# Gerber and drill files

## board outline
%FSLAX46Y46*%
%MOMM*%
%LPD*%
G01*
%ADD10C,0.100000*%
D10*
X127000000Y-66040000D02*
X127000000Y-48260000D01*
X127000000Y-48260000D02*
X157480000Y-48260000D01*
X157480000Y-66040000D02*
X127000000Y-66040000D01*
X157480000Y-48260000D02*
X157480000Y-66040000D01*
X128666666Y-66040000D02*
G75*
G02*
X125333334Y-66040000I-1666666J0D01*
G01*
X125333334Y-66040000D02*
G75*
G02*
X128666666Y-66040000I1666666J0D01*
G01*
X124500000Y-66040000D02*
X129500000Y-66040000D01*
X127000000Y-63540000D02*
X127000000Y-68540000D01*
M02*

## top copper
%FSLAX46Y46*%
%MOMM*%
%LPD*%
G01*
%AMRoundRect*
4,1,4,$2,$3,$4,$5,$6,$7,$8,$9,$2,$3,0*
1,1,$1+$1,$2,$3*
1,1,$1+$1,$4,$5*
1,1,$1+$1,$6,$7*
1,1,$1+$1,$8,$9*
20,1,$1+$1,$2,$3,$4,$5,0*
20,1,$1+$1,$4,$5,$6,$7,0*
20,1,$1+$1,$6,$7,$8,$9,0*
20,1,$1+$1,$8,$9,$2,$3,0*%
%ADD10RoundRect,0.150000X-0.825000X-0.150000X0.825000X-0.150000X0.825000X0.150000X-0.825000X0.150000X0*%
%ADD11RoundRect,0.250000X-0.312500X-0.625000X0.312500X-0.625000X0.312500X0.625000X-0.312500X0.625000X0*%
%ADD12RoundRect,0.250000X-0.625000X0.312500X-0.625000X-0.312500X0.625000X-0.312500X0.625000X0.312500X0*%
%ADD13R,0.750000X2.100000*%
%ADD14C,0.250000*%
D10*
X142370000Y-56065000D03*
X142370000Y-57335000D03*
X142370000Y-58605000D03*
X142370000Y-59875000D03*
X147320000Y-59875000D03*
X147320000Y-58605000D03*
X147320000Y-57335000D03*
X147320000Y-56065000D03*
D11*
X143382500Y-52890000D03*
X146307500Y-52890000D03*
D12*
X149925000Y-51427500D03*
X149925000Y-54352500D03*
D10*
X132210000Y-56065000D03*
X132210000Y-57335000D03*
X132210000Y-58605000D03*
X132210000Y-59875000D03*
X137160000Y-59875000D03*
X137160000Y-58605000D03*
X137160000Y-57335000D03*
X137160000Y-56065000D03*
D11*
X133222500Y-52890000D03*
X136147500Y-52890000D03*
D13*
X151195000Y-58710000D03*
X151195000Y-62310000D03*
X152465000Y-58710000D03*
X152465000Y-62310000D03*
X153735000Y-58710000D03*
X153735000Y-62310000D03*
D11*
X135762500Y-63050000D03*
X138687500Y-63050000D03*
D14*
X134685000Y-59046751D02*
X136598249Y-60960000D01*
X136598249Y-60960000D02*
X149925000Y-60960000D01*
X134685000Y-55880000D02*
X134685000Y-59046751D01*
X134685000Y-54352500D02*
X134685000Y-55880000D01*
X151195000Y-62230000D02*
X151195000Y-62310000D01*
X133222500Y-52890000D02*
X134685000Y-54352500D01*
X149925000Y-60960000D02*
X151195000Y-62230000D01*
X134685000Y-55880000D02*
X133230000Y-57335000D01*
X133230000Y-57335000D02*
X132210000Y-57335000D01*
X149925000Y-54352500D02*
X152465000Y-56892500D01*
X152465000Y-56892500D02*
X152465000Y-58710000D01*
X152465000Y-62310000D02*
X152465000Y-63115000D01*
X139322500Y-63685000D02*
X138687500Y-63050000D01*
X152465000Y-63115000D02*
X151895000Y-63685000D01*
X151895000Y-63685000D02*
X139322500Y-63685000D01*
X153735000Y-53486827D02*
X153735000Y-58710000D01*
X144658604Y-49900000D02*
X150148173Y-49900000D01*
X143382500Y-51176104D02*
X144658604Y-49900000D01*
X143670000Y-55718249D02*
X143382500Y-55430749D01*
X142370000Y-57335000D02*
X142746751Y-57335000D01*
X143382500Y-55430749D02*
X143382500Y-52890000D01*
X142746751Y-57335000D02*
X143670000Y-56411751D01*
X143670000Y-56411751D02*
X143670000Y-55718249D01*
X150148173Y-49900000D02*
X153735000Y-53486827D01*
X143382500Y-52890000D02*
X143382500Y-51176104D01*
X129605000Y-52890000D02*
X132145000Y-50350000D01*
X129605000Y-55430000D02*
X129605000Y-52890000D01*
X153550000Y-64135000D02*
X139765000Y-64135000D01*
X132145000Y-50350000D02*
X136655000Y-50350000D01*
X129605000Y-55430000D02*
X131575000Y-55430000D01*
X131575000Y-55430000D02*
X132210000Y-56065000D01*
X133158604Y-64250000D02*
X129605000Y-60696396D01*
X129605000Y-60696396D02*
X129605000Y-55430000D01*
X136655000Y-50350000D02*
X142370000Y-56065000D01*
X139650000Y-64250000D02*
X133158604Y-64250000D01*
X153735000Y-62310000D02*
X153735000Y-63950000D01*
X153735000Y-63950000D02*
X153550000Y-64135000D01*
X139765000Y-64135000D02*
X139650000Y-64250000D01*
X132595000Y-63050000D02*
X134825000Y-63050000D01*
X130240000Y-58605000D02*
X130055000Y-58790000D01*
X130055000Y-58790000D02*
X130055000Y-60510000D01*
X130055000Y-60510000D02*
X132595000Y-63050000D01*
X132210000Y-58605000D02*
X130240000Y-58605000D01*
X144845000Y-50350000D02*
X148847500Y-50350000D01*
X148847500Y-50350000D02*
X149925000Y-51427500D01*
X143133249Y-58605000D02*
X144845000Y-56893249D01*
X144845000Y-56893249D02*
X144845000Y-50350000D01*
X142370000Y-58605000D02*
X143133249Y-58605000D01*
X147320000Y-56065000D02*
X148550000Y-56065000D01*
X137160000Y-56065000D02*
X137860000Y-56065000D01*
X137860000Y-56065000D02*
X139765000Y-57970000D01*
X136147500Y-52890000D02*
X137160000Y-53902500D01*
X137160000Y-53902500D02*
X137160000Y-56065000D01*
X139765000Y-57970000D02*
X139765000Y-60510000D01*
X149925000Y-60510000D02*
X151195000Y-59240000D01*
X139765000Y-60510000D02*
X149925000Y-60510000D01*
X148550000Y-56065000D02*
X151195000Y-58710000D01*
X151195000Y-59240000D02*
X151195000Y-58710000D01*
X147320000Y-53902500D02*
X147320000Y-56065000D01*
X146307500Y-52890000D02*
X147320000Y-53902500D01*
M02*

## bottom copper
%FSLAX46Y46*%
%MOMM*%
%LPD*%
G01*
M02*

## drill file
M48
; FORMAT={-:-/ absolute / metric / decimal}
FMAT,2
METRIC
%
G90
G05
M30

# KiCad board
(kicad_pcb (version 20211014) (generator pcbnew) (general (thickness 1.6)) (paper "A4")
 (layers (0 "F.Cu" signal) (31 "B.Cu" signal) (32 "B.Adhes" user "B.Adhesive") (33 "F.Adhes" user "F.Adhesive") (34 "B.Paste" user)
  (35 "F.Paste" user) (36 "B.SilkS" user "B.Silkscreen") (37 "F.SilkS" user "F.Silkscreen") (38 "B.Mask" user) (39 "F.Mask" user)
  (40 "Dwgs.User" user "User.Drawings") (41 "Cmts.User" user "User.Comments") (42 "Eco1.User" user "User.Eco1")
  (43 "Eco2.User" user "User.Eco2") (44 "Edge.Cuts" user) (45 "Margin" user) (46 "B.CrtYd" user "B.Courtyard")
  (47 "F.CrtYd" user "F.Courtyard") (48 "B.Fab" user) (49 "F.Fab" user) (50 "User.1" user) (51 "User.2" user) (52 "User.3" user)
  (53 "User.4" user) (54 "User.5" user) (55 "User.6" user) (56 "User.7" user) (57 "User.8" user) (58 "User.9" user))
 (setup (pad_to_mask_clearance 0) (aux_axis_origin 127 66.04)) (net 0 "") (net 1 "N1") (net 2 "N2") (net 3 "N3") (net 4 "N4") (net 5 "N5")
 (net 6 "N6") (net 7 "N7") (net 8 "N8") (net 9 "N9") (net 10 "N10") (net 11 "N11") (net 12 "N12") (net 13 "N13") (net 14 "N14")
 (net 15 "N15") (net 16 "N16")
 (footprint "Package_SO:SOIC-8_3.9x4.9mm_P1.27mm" (layer "F.Cu") (at 144.845 57.97)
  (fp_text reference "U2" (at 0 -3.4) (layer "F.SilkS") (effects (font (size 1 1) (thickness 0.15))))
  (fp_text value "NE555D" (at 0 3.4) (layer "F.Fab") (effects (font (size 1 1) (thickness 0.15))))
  (pad "1" smd roundrect (at -2.475 -1.905) (size 1.95 0.6) (layers "F.Cu" "F.Paste" "F.Mask") (roundrect_rratio 0.25) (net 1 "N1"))
  (pad "2" smd roundrect (at -2.475 -0.635) (size 1.95 0.6) (layers "F.Cu" "F.Paste" "F.Mask") (roundrect_rratio 0.25) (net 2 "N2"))
  (pad "3" smd roundrect (at -2.475 0.635) (size 1.95 0.6) (layers "F.Cu" "F.Paste" "F.Mask") (roundrect_rratio 0.25) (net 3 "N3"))
  (pad "4" smd roundrect (at -2.475 1.905) (size 1.95 0.6) (layers "F.Cu" "F.Paste" "F.Mask") (roundrect_rratio 0.25) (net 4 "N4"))
  (pad "5" smd roundrect (at 2.475 1.905) (size 1.95 0.6) (layers "F.Cu" "F.Paste" "F.Mask") (roundrect_rratio 0.25) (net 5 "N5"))
  (pad "6" smd roundrect (at 2.475 0.635) (size 1.95 0.6) (layers "F.Cu" "F.Paste" "F.Mask") (roundrect_rratio 0.25) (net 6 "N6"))
  (pad "7" smd roundrect (at 2.475 -0.635) (size 1.95 0.6) (layers "F.Cu" "F.Paste" "F.Mask") (roundrect_rratio 0.25) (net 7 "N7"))
  (pad "8" smd roundrect (at 2.475 -1.905) (size 1.95 0.6) (layers "F.Cu" "F.Paste" "F.Mask") (roundrect_rratio 0.25) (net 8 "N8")))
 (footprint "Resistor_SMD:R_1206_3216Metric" (layer "F.Cu") (at 144.845 52.89)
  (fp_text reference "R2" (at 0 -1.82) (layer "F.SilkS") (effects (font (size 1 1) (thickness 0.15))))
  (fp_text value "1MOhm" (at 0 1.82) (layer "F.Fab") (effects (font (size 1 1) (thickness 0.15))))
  (pad "1" smd roundrect (at -1.4625 0) (size 1.125 1.75) (layers "F.Cu" "F.Paste" "F.Mask") (roundrect_rratio 0.222222) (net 2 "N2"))
  (pad "2" smd roundrect (at 1.4625 0) (size 1.125 1.75) (layers "F.Cu" "F.Paste" "F.Mask") (roundrect_rratio 0.222222) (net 8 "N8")))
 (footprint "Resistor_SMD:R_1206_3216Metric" (layer "F.Cu") (at 149.925 52.89 -90)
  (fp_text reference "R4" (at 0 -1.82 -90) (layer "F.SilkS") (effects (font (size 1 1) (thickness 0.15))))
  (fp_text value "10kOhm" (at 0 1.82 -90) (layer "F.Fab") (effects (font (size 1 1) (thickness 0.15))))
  (pad "1" smd roundrect (at -1.4625 0 270) (size 1.125 1.75) (layers "F.Cu" "F.Paste" "F.Mask") (roundrect_rratio 0.222222) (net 3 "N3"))
  (pad "2" smd roundrect (at 1.4625 0 270) (size 1.125 1.75) (layers "F.Cu" "F.Paste" "F.Mask") (roundrect_rratio 0.222222) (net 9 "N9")))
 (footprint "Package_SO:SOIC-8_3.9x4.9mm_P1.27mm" (layer "F.Cu") (at 134.685 57.97)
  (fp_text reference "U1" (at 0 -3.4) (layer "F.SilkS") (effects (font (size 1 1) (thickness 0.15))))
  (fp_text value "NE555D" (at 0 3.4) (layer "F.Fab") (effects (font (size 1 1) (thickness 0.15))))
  (pad "1" smd roundrect (at -2.475 -1.905) (size 1.95 0.6) (layers "F.Cu" "F.Paste" "F.Mask") (roundrect_rratio 0.25) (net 1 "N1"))
  (pad "2" smd roundrect (at -2.475 -0.635) (size 1.95 0.6) (layers "F.Cu" "F.Paste" "F.Mask") (roundrect_rratio 0.25) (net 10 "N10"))
  (pad "3" smd roundrect (at -2.475 0.635) (size 1.95 0.6) (layers "F.Cu" "F.Paste" "F.Mask") (roundrect_rratio 0.25) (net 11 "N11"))
  (pad "4" smd roundrect (at -2.475 1.905) (size 1.95 0.6) (layers "F.Cu" "F.Paste" "F.Mask") (roundrect_rratio 0.25) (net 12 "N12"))
  (pad "5" smd roundrect (at 2.475 1.905) (size 1.95 0.6) (layers "F.Cu" "F.Paste" "F.Mask") (roundrect_rratio 0.25) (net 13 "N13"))
  (pad "6" smd roundrect (at 2.475 0.635) (size 1.95 0.6) (layers "F.Cu" "F.Paste" "F.Mask") (roundrect_rratio 0.25) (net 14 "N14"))
  (pad "7" smd roundrect (at 2.475 -0.635) (size 1.95 0.6) (layers "F.Cu" "F.Paste" "F.Mask") (roundrect_rratio 0.25) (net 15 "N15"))
  (pad "8" smd roundrect (at 2.475 -1.905) (size 1.95 0.6) (layers "F.Cu" "F.Paste" "F.Mask") (roundrect_rratio 0.25) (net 8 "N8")))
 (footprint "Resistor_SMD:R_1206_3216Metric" (layer "F.Cu") (at 134.685 52.89)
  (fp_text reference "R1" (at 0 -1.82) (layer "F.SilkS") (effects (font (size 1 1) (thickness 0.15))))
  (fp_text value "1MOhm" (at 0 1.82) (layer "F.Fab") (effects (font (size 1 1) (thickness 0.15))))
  (pad "1" smd roundrect (at -1.4625 0) (size 1.125 1.75) (layers "F.Cu" "F.Paste" "F.Mask") (roundrect_rratio 0.222222) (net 10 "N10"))
  (pad "2" smd roundrect (at 1.4625 0) (size 1.125 1.75) (layers "F.Cu" "F.Paste" "F.Mask") (roundrect_rratio 0.222222) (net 8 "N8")))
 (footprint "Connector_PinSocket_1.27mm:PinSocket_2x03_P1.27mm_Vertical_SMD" (layer "F.Cu") (at 152.465 60.51 90)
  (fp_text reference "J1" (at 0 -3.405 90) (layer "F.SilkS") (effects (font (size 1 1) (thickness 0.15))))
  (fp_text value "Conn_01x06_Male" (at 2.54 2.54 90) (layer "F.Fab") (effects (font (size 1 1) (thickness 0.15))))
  (pad "1" smd rect (at 1.8 -1.27 90) (size 2.1 0.75) (layers "F.Cu" "F.Paste" "F.Mask") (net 8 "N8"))
  (pad "2" smd rect (at -1.8 -1.27 90) (size 2.1 0.75) (layers "F.Cu" "F.Paste" "F.Mask") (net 10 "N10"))
  (pad "3" smd rect (at 1.8 0 90) (size 2.1 0.75) (layers "F.Cu" "F.Paste" "F.Mask") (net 9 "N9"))
  (pad "4" smd rect (at -1.8 0 90) (size 2.1 0.75) (layers "F.Cu" "F.Paste" "F.Mask") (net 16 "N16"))
  (pad "5" smd rect (at 1.8 1.27 90) (size 2.1 0.75) (layers "F.Cu" "F.Paste" "F.Mask") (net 2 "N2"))
  (pad "6" smd rect (at -1.8 1.27 90) (size 2.1 0.75) (layers "F.Cu" "F.Paste" "F.Mask") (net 1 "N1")))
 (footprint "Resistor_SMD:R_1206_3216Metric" (layer "F.Cu") (at 137.225 63.05)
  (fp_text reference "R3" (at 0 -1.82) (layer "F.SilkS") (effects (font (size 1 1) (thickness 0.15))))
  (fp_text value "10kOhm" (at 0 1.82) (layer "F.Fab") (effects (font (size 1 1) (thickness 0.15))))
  (pad "1" smd roundrect (at -1.4625 0) (size 1.125 1.75) (layers "F.Cu" "F.Paste" "F.Mask") (roundrect_rratio 0.222222) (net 11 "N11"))
  (pad "2" smd roundrect (at 1.4625 0) (size 1.125 1.75) (layers "F.Cu" "F.Paste" "F.Mask") (roundrect_rratio 0.222222) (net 16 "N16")))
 (gr_line (start 127 66.04) (end 127 48.26) (layer "Edge.Cuts") (width 0.1))
 (gr_line (start 127 48.26) (end 157.48 48.26) (layer "Edge.Cuts") (width 0.1))
 (gr_line (start 157.48 66.04) (end 127 66.04) (layer "Edge.Cuts") (width 0.1))
 (gr_line (start 157.48 48.26) (end 157.48 66.04) (layer "Edge.Cuts") (width 0.1))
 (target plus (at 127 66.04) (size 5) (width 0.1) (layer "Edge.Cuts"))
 (segment (start 134.685 59.046751) (end 136.598249 60.96) (width 0.25) (layer "F.Cu") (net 10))
 (segment (start 136.598249 60.96) (end 149.925 60.96) (width 0.25) (layer "F.Cu") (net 10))
 (segment (start 134.685 55.88) (end 134.685 59.046751) (width 0.25) (layer "F.Cu") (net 10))
 (segment (start 134.685 54.3525) (end 134.685 55.88) (width 0.25) (layer "F.Cu") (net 10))
 (segment (start 151.195 62.23) (end 151.195 62.31) (width 0.25) (layer "F.Cu") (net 10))
 (segment (start 133.2225 52.89) (end 134.685 54.3525) (width 0.25) (layer "F.Cu") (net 10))
 (segment (start 149.925 60.96) (end 151.195 62.23) (width 0.25) (layer "F.Cu") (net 10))
 (segment (start 134.685 55.88) (end 133.23 57.335) (width 0.25) (layer "F.Cu") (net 10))
 (segment (start 133.23 57.335) (end 132.21 57.335) (width 0.25) (layer "F.Cu") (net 10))
 (segment (start 149.925 54.3525) (end 152.465 56.8925) (width 0.25) (layer "F.Cu") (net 9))
 (segment (start 152.465 56.8925) (end 152.465 58.71) (width 0.25) (layer "F.Cu") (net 9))
 (segment (start 152.465 62.31) (end 152.465 63.115) (width 0.25) (layer "F.Cu") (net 16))
 (segment (start 139.3225 63.685) (end 138.6875 63.05) (width 0.25) (layer "F.Cu") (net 16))
 (segment (start 152.465 63.115) (end 151.895 63.685) (width 0.25) (layer "F.Cu") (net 16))
 (segment (start 151.895 63.685) (end 139.3225 63.685) (width 0.25) (layer "F.Cu") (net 16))
 (segment (start 153.735 53.486827) (end 153.735 58.71) (width 0.25) (layer "F.Cu") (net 2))
 (segment (start 144.658604 49.9) (end 150.148173 49.9) (width 0.25) (layer "F.Cu") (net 2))
 (segment (start 143.3825 51.176104) (end 144.658604 49.9) (width 0.25) (layer "F.Cu") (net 2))
 (segment (start 143.67 55.718249) (end 143.3825 55.430749) (width 0.25) (layer "F.Cu") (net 2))
 (segment (start 142.37 57.335) (end 142.746751 57.335) (width 0.25) (layer "F.Cu") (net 2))
 (segment (start 143.3825 55.430749) (end 143.3825 52.89) (width 0.25) (layer "F.Cu") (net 2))
 (segment (start 142.746751 57.335) (end 143.67 56.411751) (width 0.25) (layer "F.Cu") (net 2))
 (segment (start 143.67 56.411751) (end 143.67 55.718249) (width 0.25) (layer "F.Cu") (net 2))
 (segment (start 150.148173 49.9) (end 153.735 53.486827) (width 0.25) (layer "F.Cu") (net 2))
 (segment (start 143.3825 52.89) (end 143.3825 51.176104) (width 0.25) (layer "F.Cu") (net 2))
 (segment (start 129.605 52.89) (end 132.145 50.35) (width 0.25) (layer "F.Cu") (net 1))
 (segment (start 129.605 55.43) (end 129.605 52.89) (width 0.25) (layer "F.Cu") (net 1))
 (segment (start 153.55 64.135) (end 139.765 64.135) (width 0.25) (layer "F.Cu") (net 1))
 (segment (start 132.145 50.35) (end 136.655 50.35) (width 0.25) (layer "F.Cu") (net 1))
 (segment (start 129.605 55.43) (end 131.575 55.43) (width 0.25) (layer "F.Cu") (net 1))
 (segment (start 131.575 55.43) (end 132.21 56.065) (width 0.25) (layer "F.Cu") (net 1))
 (segment (start 133.158604 64.25) (end 129.605 60.696396) (width 0.25) (layer "F.Cu") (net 1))
 (segment (start 129.605 60.696396) (end 129.605 55.43) (width 0.25) (layer "F.Cu") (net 1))
 (segment (start 136.655 50.35) (end 142.37 56.065) (width 0.25) (layer "F.Cu") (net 1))
 (segment (start 139.65 64.25) (end 133.158604 64.25) (width 0.25) (layer "F.Cu") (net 1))
 (segment (start 153.735 62.31) (end 153.735 63.95) (width 0.25) (layer "F.Cu") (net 1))
 (segment (start 153.735 63.95) (end 153.55 64.135) (width 0.25) (layer "F.Cu") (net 1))
 (segment (start 139.765 64.135) (end 139.65 64.25) (width 0.25) (layer "F.Cu") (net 1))
 (segment (start 132.595 63.05) (end 134.825 63.05) (width 0.25) (layer "F.Cu") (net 11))
 (segment (start 130.24 58.605) (end 130.055 58.79) (width 0.25) (layer "F.Cu") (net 11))
 (segment (start 130.055 58.79) (end 130.055 60.51) (width 0.25) (layer "F.Cu") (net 11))
 (segment (start 130.055 60.51) (end 132.595 63.05) (width 0.25) (layer "F.Cu") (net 11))
 (segment (start 132.21 58.605) (end 130.24 58.605) (width 0.25) (layer "F.Cu") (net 11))
 (segment (start 144.845 50.35) (end 148.8475 50.35) (width 0.25) (layer "F.Cu") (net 3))
 (segment (start 148.8475 50.35) (end 149.925 51.4275) (width 0.25) (layer "F.Cu") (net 3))
 (segment (start 143.133249 58.605) (end 144.845 56.893249) (width 0.25) (layer "F.Cu") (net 3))
 (segment (start 144.845 56.893249) (end 144.845 50.35) (width 0.25) (layer "F.Cu") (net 3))
 (segment (start 142.37 58.605) (end 143.133249 58.605) (width 0.25) (layer "F.Cu") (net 3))
 (segment (start 147.32 56.065) (end 148.55 56.065) (width 0.25) (layer "F.Cu") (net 8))
 (segment (start 137.16 56.065) (end 137.86 56.065) (width 0.25) (layer "F.Cu") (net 8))
 (segment (start 137.86 56.065) (end 139.765 57.97) (width 0.25) (layer "F.Cu") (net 8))
 (segment (start 136.1475 52.89) (end 137.16 53.9025) (width 0.25) (layer "F.Cu") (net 8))
 (segment (start 137.16 53.9025) (end 137.16 56.065) (width 0.25) (layer "F.Cu") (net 8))
 (segment (start 139.765 57.97) (end 139.765 60.51) (width 0.25) (layer "F.Cu") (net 8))
 (segment (start 149.925 60.51) (end 151.195 59.24) (width 0.25) (layer "F.Cu") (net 8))
 (segment (start 139.765 60.51) (end 149.925 60.51) (width 0.25) (layer "F.Cu") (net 8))
 (segment (start 148.55 56.065) (end 151.195 58.71) (width 0.25) (layer "F.Cu") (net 8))
 (segment (start 151.195 59.24) (end 151.195 58.71) (width 0.25) (layer "F.Cu") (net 8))
 (segment (start 147.32 53.9025) (end 147.32 56.065) (width 0.25) (layer "F.Cu") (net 8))
 (segment (start 146.3075 52.89) (end 147.32 53.9025) (width 0.25) (layer "F.Cu") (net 8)))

